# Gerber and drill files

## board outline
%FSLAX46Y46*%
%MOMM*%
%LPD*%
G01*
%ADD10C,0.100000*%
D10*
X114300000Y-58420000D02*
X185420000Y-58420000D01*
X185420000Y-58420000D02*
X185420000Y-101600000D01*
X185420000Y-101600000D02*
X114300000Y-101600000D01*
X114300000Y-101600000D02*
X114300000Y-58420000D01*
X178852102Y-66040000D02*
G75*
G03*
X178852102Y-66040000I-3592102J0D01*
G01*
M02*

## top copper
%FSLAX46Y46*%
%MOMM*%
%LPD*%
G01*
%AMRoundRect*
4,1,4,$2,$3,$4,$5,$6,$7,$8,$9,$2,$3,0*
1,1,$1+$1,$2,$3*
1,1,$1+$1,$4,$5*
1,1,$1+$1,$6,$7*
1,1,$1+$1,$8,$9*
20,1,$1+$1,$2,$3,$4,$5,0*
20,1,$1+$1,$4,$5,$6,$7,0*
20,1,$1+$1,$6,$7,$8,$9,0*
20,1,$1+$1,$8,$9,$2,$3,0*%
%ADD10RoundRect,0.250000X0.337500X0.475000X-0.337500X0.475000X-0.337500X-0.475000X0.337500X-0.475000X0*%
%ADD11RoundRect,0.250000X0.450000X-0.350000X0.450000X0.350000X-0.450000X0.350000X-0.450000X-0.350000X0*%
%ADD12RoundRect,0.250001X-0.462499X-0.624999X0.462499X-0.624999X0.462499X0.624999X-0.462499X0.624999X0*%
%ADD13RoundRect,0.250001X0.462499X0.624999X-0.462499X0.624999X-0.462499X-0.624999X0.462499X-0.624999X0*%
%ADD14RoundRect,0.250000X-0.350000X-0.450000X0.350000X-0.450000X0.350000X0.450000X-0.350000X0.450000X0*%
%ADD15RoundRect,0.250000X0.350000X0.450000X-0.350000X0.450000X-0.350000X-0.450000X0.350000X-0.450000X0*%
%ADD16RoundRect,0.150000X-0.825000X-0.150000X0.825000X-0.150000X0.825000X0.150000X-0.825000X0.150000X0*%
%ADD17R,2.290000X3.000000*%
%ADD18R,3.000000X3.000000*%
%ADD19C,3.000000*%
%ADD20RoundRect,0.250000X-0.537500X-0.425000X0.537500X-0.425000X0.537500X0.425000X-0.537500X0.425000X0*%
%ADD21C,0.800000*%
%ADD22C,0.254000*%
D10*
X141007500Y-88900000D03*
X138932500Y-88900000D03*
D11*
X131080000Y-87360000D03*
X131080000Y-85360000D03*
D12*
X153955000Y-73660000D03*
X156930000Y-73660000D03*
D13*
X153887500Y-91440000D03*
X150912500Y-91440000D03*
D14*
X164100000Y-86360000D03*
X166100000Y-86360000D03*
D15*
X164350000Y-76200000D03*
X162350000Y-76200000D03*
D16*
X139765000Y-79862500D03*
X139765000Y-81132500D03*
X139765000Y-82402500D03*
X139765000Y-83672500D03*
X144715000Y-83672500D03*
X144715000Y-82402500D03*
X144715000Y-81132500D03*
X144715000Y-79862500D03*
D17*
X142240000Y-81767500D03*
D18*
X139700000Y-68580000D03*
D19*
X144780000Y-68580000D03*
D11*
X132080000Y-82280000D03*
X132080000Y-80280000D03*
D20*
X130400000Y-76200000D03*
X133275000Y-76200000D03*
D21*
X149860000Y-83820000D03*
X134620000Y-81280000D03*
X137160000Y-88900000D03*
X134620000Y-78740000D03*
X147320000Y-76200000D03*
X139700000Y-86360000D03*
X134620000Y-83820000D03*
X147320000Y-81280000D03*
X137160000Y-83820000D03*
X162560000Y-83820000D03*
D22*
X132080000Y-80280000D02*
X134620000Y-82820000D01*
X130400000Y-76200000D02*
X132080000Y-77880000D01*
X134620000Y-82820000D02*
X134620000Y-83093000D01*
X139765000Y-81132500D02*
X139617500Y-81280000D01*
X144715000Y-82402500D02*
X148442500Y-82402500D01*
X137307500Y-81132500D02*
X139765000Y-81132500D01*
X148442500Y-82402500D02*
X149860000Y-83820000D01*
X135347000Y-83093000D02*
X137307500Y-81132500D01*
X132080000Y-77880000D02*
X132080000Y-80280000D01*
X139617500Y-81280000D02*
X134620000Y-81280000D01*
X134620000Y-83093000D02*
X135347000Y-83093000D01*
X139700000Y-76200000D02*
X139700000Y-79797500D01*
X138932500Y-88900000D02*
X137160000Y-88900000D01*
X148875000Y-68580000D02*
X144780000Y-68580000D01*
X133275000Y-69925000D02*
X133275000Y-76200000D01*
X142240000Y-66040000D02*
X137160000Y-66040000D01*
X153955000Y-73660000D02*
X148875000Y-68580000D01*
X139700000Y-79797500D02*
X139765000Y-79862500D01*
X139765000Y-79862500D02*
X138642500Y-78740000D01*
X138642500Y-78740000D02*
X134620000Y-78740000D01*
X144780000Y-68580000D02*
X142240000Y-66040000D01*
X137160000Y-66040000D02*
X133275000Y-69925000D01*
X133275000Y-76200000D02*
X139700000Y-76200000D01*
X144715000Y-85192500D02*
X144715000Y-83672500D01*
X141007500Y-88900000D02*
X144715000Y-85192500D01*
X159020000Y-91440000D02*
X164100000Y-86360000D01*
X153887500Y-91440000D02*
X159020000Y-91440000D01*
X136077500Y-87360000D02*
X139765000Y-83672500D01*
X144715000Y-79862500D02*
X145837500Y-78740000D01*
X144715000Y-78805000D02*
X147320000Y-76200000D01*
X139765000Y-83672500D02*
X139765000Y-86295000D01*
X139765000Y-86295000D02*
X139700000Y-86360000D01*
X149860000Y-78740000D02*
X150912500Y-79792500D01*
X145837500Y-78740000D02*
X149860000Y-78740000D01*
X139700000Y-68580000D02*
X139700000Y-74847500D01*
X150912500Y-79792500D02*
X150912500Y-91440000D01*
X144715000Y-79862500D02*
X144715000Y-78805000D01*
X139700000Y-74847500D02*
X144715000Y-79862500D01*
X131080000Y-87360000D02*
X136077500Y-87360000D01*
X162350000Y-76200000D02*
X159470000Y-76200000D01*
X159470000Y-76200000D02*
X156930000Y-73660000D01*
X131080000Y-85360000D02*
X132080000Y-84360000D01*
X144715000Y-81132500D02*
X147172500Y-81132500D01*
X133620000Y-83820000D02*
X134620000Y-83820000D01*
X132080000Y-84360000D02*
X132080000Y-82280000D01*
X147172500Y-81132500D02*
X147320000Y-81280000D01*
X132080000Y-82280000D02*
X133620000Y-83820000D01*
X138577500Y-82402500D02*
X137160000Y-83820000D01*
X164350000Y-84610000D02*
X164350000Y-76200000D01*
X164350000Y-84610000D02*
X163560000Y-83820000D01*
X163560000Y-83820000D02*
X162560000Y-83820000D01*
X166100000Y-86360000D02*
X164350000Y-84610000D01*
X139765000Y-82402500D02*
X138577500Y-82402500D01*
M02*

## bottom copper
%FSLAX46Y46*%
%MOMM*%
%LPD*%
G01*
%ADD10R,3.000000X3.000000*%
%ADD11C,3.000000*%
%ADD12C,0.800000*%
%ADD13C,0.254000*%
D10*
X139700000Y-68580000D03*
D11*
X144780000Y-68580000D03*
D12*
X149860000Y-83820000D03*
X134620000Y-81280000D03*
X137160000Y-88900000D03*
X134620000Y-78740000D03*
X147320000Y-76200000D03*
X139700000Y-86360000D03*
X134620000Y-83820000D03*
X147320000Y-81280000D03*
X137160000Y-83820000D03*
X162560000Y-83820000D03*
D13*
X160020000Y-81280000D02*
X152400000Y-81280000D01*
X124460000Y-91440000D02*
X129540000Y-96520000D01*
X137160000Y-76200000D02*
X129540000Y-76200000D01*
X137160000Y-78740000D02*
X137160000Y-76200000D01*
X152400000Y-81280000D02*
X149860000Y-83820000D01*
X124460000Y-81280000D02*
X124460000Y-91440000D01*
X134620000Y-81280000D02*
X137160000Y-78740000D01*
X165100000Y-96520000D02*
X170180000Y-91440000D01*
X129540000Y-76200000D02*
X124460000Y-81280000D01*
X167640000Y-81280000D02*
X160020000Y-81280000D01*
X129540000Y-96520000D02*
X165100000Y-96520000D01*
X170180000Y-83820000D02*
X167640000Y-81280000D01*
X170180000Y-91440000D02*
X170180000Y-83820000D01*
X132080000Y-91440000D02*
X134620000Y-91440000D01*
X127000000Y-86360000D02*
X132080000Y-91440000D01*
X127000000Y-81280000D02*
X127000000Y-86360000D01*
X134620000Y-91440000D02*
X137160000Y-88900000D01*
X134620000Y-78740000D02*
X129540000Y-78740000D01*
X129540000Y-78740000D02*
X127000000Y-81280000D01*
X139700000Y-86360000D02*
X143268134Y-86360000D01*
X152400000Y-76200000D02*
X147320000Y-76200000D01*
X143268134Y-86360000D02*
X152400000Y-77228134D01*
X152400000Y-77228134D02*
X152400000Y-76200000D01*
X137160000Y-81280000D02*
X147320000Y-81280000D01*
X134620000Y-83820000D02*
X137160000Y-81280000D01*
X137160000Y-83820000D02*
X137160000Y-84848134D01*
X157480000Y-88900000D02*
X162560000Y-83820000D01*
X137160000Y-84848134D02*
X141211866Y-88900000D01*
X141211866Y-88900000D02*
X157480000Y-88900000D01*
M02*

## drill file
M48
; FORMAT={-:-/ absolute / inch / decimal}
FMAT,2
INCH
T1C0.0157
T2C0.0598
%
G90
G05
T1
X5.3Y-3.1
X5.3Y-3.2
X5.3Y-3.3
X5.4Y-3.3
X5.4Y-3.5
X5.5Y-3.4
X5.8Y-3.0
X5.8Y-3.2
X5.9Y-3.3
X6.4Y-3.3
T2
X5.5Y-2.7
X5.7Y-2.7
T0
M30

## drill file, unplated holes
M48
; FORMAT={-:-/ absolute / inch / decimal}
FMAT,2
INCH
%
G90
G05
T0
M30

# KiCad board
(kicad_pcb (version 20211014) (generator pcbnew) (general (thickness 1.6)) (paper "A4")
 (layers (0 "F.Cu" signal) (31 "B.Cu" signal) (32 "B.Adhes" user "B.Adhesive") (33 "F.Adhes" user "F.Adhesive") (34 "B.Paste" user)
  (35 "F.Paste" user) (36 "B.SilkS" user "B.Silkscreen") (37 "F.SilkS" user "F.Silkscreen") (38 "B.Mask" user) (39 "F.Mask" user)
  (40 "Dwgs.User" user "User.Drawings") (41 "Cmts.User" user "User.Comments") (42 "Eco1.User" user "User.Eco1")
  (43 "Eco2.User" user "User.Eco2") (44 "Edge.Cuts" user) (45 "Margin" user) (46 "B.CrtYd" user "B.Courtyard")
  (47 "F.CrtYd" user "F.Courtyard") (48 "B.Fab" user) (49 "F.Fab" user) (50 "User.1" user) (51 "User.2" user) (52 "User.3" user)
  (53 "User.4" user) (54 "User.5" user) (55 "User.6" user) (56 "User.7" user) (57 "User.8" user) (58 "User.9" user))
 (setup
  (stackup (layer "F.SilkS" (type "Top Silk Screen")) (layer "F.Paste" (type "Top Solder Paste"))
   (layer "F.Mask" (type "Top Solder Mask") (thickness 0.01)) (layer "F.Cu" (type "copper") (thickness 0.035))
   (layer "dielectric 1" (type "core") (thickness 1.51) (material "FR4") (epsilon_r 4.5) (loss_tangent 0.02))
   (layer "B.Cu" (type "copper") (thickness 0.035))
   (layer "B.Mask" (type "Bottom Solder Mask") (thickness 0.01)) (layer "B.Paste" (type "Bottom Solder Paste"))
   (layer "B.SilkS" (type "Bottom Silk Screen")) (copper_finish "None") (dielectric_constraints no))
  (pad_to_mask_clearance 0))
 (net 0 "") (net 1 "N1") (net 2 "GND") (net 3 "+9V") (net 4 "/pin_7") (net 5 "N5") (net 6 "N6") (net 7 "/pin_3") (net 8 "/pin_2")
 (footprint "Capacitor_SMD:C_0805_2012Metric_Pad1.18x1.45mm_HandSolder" (layer "F.Cu") (at 139.97 88.9 180)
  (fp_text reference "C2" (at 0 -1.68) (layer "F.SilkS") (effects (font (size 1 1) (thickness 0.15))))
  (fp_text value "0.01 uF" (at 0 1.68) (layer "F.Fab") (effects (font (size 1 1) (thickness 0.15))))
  (pad "1" smd roundrect (at -1.0375 0 180) (size 1.175 1.45) (layers "F.Cu" "F.Paste" "F.Mask") (roundrect_rratio 0.2127659574)
   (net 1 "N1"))
  (pad "2" smd roundrect (at 1.0375 0 180) (size 1.175 1.45) (layers "F.Cu" "F.Paste" "F.Mask") (roundrect_rratio 0.2127659574)
   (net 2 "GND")))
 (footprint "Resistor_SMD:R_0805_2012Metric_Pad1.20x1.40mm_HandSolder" (layer "F.Cu") (at 131.08 86.36 90)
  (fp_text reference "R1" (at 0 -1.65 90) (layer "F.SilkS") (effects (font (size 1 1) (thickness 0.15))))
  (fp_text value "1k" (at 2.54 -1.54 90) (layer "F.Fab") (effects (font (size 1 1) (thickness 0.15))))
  (pad "1" smd roundrect (at -1 0 90) (size 1.2 1.4) (layers "F.Cu" "F.Paste" "F.Mask") (roundrect_rratio 0.2083333333) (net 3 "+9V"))
  (pad "2" smd roundrect (at 1 0 90) (size 1.2 1.4) (layers "F.Cu" "F.Paste" "F.Mask") (roundrect_rratio 0.2083333333) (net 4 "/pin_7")))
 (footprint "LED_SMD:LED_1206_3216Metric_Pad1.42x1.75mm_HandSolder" (layer "F.Cu") (at 155.4425 73.66)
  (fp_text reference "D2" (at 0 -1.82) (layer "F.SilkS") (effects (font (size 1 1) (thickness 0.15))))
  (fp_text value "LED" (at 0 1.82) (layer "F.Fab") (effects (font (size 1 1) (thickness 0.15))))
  (pad "1" smd roundrect (at -1.4875 0) (size 1.425 1.75) (layers "F.Cu" "F.Paste" "F.Mask") (roundrect_rratio 0.1754392982) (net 2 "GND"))
  (pad "2" smd roundrect (at 1.4875 0) (size 1.425 1.75) (layers "F.Cu" "F.Paste" "F.Mask") (roundrect_rratio 0.1754392982) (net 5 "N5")))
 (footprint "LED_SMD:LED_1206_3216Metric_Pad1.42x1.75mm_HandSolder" (layer "F.Cu") (at 152.4 91.44 180)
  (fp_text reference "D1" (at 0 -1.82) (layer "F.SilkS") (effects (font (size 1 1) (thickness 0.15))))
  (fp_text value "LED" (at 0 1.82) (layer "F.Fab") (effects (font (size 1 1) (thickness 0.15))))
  (pad "1" smd roundrect (at -1.4875 0 180) (size 1.425 1.75) (layers "F.Cu" "F.Paste" "F.Mask") (roundrect_rratio 0.1754392982)
   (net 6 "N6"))
  (pad "2" smd roundrect (at 1.4875 0 180) (size 1.425 1.75) (layers "F.Cu" "F.Paste" "F.Mask") (roundrect_rratio 0.1754392982)
   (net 3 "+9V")))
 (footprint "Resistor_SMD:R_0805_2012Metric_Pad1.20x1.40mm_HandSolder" (layer "F.Cu") (at 165.1 86.36)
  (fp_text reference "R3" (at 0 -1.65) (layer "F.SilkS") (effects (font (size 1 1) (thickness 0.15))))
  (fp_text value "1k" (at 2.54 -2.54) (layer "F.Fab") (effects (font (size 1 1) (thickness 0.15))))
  (pad "1" smd roundrect (at -1 0) (size 1.2 1.4) (layers "F.Cu" "F.Paste" "F.Mask") (roundrect_rratio 0.2083333333) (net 6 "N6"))
  (pad "2" smd roundrect (at 1 0) (size 1.2 1.4) (layers "F.Cu" "F.Paste" "F.Mask") (roundrect_rratio 0.2083333333) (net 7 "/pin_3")))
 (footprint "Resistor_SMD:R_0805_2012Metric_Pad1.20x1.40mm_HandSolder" (layer "F.Cu") (at 163.35 76.2 180)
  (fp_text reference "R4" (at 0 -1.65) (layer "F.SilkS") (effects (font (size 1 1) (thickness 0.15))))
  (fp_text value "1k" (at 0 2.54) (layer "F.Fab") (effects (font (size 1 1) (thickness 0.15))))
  (pad "1" smd roundrect (at -1 0 180) (size 1.2 1.4) (layers "F.Cu" "F.Paste" "F.Mask") (roundrect_rratio 0.2083333333) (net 7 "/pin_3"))
  (pad "2" smd roundrect (at 1 0 180) (size 1.2 1.4) (layers "F.Cu" "F.Paste" "F.Mask") (roundrect_rratio 0.2083333333) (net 5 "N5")))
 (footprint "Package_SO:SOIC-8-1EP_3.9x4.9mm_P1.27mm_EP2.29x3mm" (layer "F.Cu") (at 142.24 81.7675)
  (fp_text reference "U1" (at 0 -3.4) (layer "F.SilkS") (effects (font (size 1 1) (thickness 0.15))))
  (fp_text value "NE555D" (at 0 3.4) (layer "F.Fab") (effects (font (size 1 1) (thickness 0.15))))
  (pad "" smd roundrect (at 0.57 0.75) (size 0.92 1.21) (layers "F.Paste") (roundrect_rratio 0.25))
  (pad "" smd roundrect (at 0.57 -0.75) (size 0.92 1.21) (layers "F.Paste") (roundrect_rratio 0.25))
  (pad "" smd roundrect (at -0.57 0.75) (size 0.92 1.21) (layers "F.Paste") (roundrect_rratio 0.25))
  (pad "" smd roundrect (at -0.57 -0.75) (size 0.92 1.21) (layers "F.Paste") (roundrect_rratio 0.25))
  (pad "1" smd roundrect (at -2.475 -1.905) (size 1.95 0.6) (layers "F.Cu" "F.Paste" "F.Mask") (roundrect_rratio 0.25) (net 2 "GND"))
  (pad "2" smd roundrect (at -2.475 -0.635) (size 1.95 0.6) (layers "F.Cu" "F.Paste" "F.Mask") (roundrect_rratio 0.25) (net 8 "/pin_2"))
  (pad "3" smd roundrect (at -2.475 0.635) (size 1.95 0.6) (layers "F.Cu" "F.Paste" "F.Mask") (roundrect_rratio 0.25) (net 7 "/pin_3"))
  (pad "4" smd roundrect (at -2.475 1.905) (size 1.95 0.6) (layers "F.Cu" "F.Paste" "F.Mask") (roundrect_rratio 0.25) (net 3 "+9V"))
  (pad "5" smd roundrect (at 2.475 1.905) (size 1.95 0.6) (layers "F.Cu" "F.Paste" "F.Mask") (roundrect_rratio 0.25) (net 1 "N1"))
  (pad "6" smd roundrect (at 2.475 0.635) (size 1.95 0.6) (layers "F.Cu" "F.Paste" "F.Mask") (roundrect_rratio 0.25) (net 8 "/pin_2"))
  (pad "7" smd roundrect (at 2.475 -0.635) (size 1.95 0.6) (layers "F.Cu" "F.Paste" "F.Mask") (roundrect_rratio 0.25) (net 4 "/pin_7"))
  (pad "8" smd roundrect (at 2.475 -1.905) (size 1.95 0.6) (layers "F.Cu" "F.Paste" "F.Mask") (roundrect_rratio 0.25) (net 3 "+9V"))
  (pad "9" smd rect (at 0 0) (size 2.29 3) (layers "F.Cu" "F.Mask")))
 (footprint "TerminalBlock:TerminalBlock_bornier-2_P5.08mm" (layer "F.Cu") (at 139.7 68.58)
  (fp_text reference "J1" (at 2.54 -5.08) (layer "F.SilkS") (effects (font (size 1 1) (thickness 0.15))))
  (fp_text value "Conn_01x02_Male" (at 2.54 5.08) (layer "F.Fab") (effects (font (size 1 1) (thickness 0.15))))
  (pad "1" thru_hole rect (at 0 0) (size 3 3) (drill 1.52) (layers *.Cu *.Mask) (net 3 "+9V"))
  (pad "2" thru_hole circle (at 5.08 0) (size 3 3) (drill 1.52) (layers *.Cu *.Mask) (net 2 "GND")))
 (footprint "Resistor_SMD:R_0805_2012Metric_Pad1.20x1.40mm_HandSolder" (layer "F.Cu") (at 132.08 81.28 90)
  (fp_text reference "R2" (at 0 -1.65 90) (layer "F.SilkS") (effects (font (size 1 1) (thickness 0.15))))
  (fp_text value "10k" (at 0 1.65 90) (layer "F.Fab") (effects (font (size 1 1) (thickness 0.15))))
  (pad "1" smd roundrect (at -1 0 90) (size 1.2 1.4) (layers "F.Cu" "F.Paste" "F.Mask") (roundrect_rratio 0.2083333333) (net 4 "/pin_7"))
  (pad "2" smd roundrect (at 1 0 90) (size 1.2 1.4) (layers "F.Cu" "F.Paste" "F.Mask") (roundrect_rratio 0.2083333333) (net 8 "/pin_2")))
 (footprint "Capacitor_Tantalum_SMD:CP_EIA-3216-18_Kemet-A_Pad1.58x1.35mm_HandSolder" (layer "F.Cu") (at 131.8375 76.2)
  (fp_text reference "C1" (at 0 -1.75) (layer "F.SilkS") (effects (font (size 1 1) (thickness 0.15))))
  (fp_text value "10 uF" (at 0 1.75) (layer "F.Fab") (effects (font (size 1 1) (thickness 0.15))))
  (pad "1" smd roundrect (at -1.4375 0) (size 1.575 1.35) (layers "F.Cu" "F.Paste" "F.Mask") (roundrect_rratio 0.1851851852)
   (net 8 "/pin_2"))
  (pad "2" smd roundrect (at 1.4375 0) (size 1.575 1.35) (layers "F.Cu" "F.Paste" "F.Mask") (roundrect_rratio 0.1851851852) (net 2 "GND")))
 (gr_rect (start 114.3 58.42) (end 185.42 101.6) (layer "Edge.Cuts") (width 0.1) (fill none))
 (gr_circle (center 175.26 66.04) (end 177.8 68.58) (layer "Edge.Cuts") (width 0.1) (fill none))
 (segment (start 132.08 80.28) (end 134.62 82.82) (width 0.254) (layer "F.Cu") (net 8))
 (segment (start 130.4 76.2) (end 132.08 77.88) (width 0.254) (layer "F.Cu") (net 8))
 (segment (start 134.62 82.82) (end 134.62 83.093) (width 0.254) (layer "F.Cu") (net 8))
 (segment (start 139.765 81.1325) (end 139.6175 81.28) (width 0.254) (layer "F.Cu") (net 8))
 (segment (start 144.715 82.4025) (end 148.4425 82.4025) (width 0.254) (layer "F.Cu") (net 8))
 (segment (start 137.3075 81.1325) (end 139.765 81.1325) (width 0.254) (layer "F.Cu") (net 8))
 (segment (start 148.4425 82.4025) (end 149.86 83.82) (width 0.254) (layer "F.Cu") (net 8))
 (segment (start 135.347 83.093) (end 137.3075 81.1325) (width 0.254) (layer "F.Cu") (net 8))
 (segment (start 132.08 77.88) (end 132.08 80.28) (width 0.254) (layer "F.Cu") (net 8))
 (segment (start 139.6175 81.28) (end 134.62 81.28) (width 0.254) (layer "F.Cu") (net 8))
 (segment (start 134.62 83.093) (end 135.347 83.093) (width 0.254) (layer "F.Cu") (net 8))
 (via (at 149.86 83.82) (size 0.8) (drill 0.4) (layers "F.Cu" "B.Cu") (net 8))
 (via (at 134.62 81.28) (size 0.8) (drill 0.4) (layers "F.Cu" "B.Cu") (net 8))
 (segment (start 160.02 81.28) (end 152.4 81.28) (width 0.254) (layer "B.Cu") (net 8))
 (segment (start 124.46 91.44) (end 129.54 96.52) (width 0.254) (layer "B.Cu") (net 8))
 (segment (start 137.16 76.2) (end 129.54 76.2) (width 0.254) (layer "B.Cu") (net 8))
 (segment (start 137.16 78.74) (end 137.16 76.2) (width 0.254) (layer "B.Cu") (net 8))
 (segment (start 152.4 81.28) (end 149.86 83.82) (width 0.254) (layer "B.Cu") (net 8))
 (segment (start 124.46 81.28) (end 124.46 91.44) (width 0.254) (layer "B.Cu") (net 8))
 (segment (start 134.62 81.28) (end 137.16 78.74) (width 0.254) (layer "B.Cu") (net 8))
 (segment (start 165.1 96.52) (end 170.18 91.44) (width 0.254) (layer "B.Cu") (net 8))
 (segment (start 129.54 76.2) (end 124.46 81.28) (width 0.254) (layer "B.Cu") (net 8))
 (segment (start 167.64 81.28) (end 160.02 81.28) (width 0.254) (layer "B.Cu") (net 8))
 (segment (start 129.54 96.52) (end 165.1 96.52) (width 0.254) (layer "B.Cu") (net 8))
 (segment (start 170.18 83.82) (end 167.64 81.28) (width 0.254) (layer "B.Cu") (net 8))
 (segment (start 170.18 91.44) (end 170.18 83.82) (width 0.254) (layer "B.Cu") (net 8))
 (segment (start 139.7 76.2) (end 139.7 79.7975) (width 0.254) (layer "F.Cu") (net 2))
 (segment (start 138.9325 88.9) (end 137.16 88.9) (width 0.254) (layer "F.Cu") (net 2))
 (segment (start 148.875 68.58) (end 144.78 68.58) (width 0.254) (layer "F.Cu") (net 2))
 (segment (start 133.275 69.925) (end 133.275 76.2) (width 0.254) (layer "F.Cu") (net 2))
 (segment (start 142.24 66.04) (end 137.16 66.04) (width 0.254) (layer "F.Cu") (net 2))
 (segment (start 153.955 73.66) (end 148.875 68.58) (width 0.254) (layer "F.Cu") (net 2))
 (segment (start 139.7 79.7975) (end 139.765 79.8625) (width 0.254) (layer "F.Cu") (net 2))
 (segment (start 139.765 79.8625) (end 138.6425 78.74) (width 0.254) (layer "F.Cu") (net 2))
 (segment (start 138.6425 78.74) (end 134.62 78.74) (width 0.254) (layer "F.Cu") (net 2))
 (segment (start 144.78 68.58) (end 142.24 66.04) (width 0.254) (layer "F.Cu") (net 2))
 (segment (start 137.16 66.04) (end 133.275 69.925) (width 0.254) (layer "F.Cu") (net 2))
 (segment (start 133.275 76.2) (end 139.7 76.2) (width 0.254) (layer "F.Cu") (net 2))
 (via (at 137.16 88.9) (size 0.8) (drill 0.4) (layers "F.Cu" "B.Cu") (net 2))
 (via (at 134.62 78.74) (size 0.8) (drill 0.4) (layers "F.Cu" "B.Cu") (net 2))
 (segment (start 132.08 91.44) (end 134.62 91.44) (width 0.254) (layer "B.Cu") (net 2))
 (segment (start 127 86.36) (end 132.08 91.44) (width 0.254) (layer "B.Cu") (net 2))
 (segment (start 127 81.28) (end 127 86.36) (width 0.254) (layer "B.Cu") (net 2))
 (segment (start 134.62 91.44) (end 137.16 88.9) (width 0.254) (layer "B.Cu") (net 2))
 (segment (start 134.62 78.74) (end 129.54 78.74) (width 0.254) (layer "B.Cu") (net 2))
 (segment (start 129.54 78.74) (end 127 81.28) (width 0.254) (layer "B.Cu") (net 2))
 (segment (start 144.715 85.1925) (end 144.715 83.6725) (width 0.254) (layer "F.Cu") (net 1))
 (segment (start 141.0075 88.9) (end 144.715 85.1925) (width 0.254) (layer "F.Cu") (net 1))
 (segment (start 159.02 91.44) (end 164.1 86.36) (width 0.254) (layer "F.Cu") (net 6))
 (segment (start 153.8875 91.44) (end 159.02 91.44) (width 0.254) (layer "F.Cu") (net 6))
 (segment (start 136.0775 87.36) (end 139.765 83.6725) (width 0.254) (layer "F.Cu") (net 3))
 (segment (start 144.715 79.8625) (end 145.8375 78.74) (width 0.254) (layer "F.Cu") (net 3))
 (segment (start 144.715 78.805) (end 147.32 76.2) (width 0.254) (layer "F.Cu") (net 3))
 (segment (start 139.765 83.6725) (end 139.765 86.295) (width 0.254) (layer "F.Cu") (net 3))
 (segment (start 139.765 86.295) (end 139.7 86.36) (width 0.254) (layer "F.Cu") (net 3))
 (segment (start 149.86 78.74) (end 150.9125 79.7925) (width 0.254) (layer "F.Cu") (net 3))
 (segment (start 145.8375 78.74) (end 149.86 78.74) (width 0.254) (layer "F.Cu") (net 3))
 (segment (start 139.7 68.58) (end 139.7 74.8475) (width 0.254) (layer "F.Cu") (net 3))
 (segment (start 150.9125 79.7925) (end 150.9125 91.44) (width 0.254) (layer "F.Cu") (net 3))
 (segment (start 144.715 79.8625) (end 144.715 78.805) (width 0.254) (layer "F.Cu") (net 3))
 (segment (start 139.7 74.8475) (end 144.715 79.8625) (width 0.254) (layer "F.Cu") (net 3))
 (segment (start 131.08 87.36) (end 136.0775 87.36) (width 0.254) (layer "F.Cu") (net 3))
 (via (at 147.32 76.2) (size 0.8) (drill 0.4) (layers "F.Cu" "B.Cu") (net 3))
 (via (at 139.7 86.36) (size 0.8) (drill 0.4) (layers "F.Cu" "B.Cu") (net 3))
 (segment (start 139.7 86.36) (end 143.268134 86.36) (width 0.254) (layer "B.Cu") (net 3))
 (segment (start 152.4 76.2) (end 147.32 76.2) (width 0.254) (layer "B.Cu") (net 3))
 (segment (start 143.268134 86.36) (end 152.4 77.228134) (width 0.254) (layer "B.Cu") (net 3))
 (segment (start 152.4 77.228134) (end 152.4 76.2) (width 0.254) (layer "B.Cu") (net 3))
 (segment (start 162.35 76.2) (end 159.47 76.2) (width 0.254) (layer "F.Cu") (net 5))
 (segment (start 159.47 76.2) (end 156.93 73.66) (width 0.254) (layer "F.Cu") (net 5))
 (segment (start 131.08 85.36) (end 132.08 84.36) (width 0.254) (layer "F.Cu") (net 4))
 (segment (start 144.715 81.1325) (end 147.1725 81.1325) (width 0.254) (layer "F.Cu") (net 4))
 (segment (start 133.62 83.82) (end 134.62 83.82) (width 0.254) (layer "F.Cu") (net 4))
 (segment (start 132.08 84.36) (end 132.08 82.28) (width 0.254) (layer "F.Cu") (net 4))
 (segment (start 147.1725 81.1325) (end 147.32 81.28) (width 0.254) (layer "F.Cu") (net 4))
 (segment (start 132.08 82.28) (end 133.62 83.82) (width 0.254) (layer "F.Cu") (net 4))
 (via (at 134.62 83.82) (size 0.8) (drill 0.4) (layers "F.Cu" "B.Cu") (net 4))
 (via (at 147.32 81.28) (size 0.8) (drill 0.4) (layers "F.Cu" "B.Cu") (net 4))
 (segment (start 137.16 81.28) (end 147.32 81.28) (width 0.254) (layer "B.Cu") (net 4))
 (segment (start 134.62 83.82) (end 137.16 81.28) (width 0.254) (layer "B.Cu") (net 4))
 (segment (start 138.5775 82.4025) (end 137.16 83.82) (width 0.254) (layer "F.Cu") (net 7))
 (segment (start 164.35 84.61) (end 164.35 76.2) (width 0.254) (layer "F.Cu") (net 7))
 (segment (start 164.35 84.61) (end 163.56 83.82) (width 0.254) (layer "F.Cu") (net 7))
 (segment (start 163.56 83.82) (end 162.56 83.82) (width 0.254) (layer "F.Cu") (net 7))
 (segment (start 166.1 86.36) (end 164.35 84.61) (width 0.254) (layer "F.Cu") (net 7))
 (segment (start 139.765 82.4025) (end 138.5775 82.4025) (width 0.254) (layer "F.Cu") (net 7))
 (via (at 137.16 83.82) (size 0.8) (drill 0.4) (layers "F.Cu" "B.Cu") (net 7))
 (via (at 162.56 83.82) (size 0.8) (drill 0.4) (layers "F.Cu" "B.Cu") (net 7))
 (segment (start 137.16 83.82) (end 137.16 84.848134) (width 0.254) (layer "B.Cu") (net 7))
 (segment (start 157.48 88.9) (end 162.56 83.82) (width 0.254) (layer "B.Cu") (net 7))
 (segment (start 137.16 84.848134) (end 141.211866 88.9) (width 0.254) (layer "B.Cu") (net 7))
 (segment (start 141.211866 88.9) (end 157.48 88.9) (width 0.254) (layer "B.Cu") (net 7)))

